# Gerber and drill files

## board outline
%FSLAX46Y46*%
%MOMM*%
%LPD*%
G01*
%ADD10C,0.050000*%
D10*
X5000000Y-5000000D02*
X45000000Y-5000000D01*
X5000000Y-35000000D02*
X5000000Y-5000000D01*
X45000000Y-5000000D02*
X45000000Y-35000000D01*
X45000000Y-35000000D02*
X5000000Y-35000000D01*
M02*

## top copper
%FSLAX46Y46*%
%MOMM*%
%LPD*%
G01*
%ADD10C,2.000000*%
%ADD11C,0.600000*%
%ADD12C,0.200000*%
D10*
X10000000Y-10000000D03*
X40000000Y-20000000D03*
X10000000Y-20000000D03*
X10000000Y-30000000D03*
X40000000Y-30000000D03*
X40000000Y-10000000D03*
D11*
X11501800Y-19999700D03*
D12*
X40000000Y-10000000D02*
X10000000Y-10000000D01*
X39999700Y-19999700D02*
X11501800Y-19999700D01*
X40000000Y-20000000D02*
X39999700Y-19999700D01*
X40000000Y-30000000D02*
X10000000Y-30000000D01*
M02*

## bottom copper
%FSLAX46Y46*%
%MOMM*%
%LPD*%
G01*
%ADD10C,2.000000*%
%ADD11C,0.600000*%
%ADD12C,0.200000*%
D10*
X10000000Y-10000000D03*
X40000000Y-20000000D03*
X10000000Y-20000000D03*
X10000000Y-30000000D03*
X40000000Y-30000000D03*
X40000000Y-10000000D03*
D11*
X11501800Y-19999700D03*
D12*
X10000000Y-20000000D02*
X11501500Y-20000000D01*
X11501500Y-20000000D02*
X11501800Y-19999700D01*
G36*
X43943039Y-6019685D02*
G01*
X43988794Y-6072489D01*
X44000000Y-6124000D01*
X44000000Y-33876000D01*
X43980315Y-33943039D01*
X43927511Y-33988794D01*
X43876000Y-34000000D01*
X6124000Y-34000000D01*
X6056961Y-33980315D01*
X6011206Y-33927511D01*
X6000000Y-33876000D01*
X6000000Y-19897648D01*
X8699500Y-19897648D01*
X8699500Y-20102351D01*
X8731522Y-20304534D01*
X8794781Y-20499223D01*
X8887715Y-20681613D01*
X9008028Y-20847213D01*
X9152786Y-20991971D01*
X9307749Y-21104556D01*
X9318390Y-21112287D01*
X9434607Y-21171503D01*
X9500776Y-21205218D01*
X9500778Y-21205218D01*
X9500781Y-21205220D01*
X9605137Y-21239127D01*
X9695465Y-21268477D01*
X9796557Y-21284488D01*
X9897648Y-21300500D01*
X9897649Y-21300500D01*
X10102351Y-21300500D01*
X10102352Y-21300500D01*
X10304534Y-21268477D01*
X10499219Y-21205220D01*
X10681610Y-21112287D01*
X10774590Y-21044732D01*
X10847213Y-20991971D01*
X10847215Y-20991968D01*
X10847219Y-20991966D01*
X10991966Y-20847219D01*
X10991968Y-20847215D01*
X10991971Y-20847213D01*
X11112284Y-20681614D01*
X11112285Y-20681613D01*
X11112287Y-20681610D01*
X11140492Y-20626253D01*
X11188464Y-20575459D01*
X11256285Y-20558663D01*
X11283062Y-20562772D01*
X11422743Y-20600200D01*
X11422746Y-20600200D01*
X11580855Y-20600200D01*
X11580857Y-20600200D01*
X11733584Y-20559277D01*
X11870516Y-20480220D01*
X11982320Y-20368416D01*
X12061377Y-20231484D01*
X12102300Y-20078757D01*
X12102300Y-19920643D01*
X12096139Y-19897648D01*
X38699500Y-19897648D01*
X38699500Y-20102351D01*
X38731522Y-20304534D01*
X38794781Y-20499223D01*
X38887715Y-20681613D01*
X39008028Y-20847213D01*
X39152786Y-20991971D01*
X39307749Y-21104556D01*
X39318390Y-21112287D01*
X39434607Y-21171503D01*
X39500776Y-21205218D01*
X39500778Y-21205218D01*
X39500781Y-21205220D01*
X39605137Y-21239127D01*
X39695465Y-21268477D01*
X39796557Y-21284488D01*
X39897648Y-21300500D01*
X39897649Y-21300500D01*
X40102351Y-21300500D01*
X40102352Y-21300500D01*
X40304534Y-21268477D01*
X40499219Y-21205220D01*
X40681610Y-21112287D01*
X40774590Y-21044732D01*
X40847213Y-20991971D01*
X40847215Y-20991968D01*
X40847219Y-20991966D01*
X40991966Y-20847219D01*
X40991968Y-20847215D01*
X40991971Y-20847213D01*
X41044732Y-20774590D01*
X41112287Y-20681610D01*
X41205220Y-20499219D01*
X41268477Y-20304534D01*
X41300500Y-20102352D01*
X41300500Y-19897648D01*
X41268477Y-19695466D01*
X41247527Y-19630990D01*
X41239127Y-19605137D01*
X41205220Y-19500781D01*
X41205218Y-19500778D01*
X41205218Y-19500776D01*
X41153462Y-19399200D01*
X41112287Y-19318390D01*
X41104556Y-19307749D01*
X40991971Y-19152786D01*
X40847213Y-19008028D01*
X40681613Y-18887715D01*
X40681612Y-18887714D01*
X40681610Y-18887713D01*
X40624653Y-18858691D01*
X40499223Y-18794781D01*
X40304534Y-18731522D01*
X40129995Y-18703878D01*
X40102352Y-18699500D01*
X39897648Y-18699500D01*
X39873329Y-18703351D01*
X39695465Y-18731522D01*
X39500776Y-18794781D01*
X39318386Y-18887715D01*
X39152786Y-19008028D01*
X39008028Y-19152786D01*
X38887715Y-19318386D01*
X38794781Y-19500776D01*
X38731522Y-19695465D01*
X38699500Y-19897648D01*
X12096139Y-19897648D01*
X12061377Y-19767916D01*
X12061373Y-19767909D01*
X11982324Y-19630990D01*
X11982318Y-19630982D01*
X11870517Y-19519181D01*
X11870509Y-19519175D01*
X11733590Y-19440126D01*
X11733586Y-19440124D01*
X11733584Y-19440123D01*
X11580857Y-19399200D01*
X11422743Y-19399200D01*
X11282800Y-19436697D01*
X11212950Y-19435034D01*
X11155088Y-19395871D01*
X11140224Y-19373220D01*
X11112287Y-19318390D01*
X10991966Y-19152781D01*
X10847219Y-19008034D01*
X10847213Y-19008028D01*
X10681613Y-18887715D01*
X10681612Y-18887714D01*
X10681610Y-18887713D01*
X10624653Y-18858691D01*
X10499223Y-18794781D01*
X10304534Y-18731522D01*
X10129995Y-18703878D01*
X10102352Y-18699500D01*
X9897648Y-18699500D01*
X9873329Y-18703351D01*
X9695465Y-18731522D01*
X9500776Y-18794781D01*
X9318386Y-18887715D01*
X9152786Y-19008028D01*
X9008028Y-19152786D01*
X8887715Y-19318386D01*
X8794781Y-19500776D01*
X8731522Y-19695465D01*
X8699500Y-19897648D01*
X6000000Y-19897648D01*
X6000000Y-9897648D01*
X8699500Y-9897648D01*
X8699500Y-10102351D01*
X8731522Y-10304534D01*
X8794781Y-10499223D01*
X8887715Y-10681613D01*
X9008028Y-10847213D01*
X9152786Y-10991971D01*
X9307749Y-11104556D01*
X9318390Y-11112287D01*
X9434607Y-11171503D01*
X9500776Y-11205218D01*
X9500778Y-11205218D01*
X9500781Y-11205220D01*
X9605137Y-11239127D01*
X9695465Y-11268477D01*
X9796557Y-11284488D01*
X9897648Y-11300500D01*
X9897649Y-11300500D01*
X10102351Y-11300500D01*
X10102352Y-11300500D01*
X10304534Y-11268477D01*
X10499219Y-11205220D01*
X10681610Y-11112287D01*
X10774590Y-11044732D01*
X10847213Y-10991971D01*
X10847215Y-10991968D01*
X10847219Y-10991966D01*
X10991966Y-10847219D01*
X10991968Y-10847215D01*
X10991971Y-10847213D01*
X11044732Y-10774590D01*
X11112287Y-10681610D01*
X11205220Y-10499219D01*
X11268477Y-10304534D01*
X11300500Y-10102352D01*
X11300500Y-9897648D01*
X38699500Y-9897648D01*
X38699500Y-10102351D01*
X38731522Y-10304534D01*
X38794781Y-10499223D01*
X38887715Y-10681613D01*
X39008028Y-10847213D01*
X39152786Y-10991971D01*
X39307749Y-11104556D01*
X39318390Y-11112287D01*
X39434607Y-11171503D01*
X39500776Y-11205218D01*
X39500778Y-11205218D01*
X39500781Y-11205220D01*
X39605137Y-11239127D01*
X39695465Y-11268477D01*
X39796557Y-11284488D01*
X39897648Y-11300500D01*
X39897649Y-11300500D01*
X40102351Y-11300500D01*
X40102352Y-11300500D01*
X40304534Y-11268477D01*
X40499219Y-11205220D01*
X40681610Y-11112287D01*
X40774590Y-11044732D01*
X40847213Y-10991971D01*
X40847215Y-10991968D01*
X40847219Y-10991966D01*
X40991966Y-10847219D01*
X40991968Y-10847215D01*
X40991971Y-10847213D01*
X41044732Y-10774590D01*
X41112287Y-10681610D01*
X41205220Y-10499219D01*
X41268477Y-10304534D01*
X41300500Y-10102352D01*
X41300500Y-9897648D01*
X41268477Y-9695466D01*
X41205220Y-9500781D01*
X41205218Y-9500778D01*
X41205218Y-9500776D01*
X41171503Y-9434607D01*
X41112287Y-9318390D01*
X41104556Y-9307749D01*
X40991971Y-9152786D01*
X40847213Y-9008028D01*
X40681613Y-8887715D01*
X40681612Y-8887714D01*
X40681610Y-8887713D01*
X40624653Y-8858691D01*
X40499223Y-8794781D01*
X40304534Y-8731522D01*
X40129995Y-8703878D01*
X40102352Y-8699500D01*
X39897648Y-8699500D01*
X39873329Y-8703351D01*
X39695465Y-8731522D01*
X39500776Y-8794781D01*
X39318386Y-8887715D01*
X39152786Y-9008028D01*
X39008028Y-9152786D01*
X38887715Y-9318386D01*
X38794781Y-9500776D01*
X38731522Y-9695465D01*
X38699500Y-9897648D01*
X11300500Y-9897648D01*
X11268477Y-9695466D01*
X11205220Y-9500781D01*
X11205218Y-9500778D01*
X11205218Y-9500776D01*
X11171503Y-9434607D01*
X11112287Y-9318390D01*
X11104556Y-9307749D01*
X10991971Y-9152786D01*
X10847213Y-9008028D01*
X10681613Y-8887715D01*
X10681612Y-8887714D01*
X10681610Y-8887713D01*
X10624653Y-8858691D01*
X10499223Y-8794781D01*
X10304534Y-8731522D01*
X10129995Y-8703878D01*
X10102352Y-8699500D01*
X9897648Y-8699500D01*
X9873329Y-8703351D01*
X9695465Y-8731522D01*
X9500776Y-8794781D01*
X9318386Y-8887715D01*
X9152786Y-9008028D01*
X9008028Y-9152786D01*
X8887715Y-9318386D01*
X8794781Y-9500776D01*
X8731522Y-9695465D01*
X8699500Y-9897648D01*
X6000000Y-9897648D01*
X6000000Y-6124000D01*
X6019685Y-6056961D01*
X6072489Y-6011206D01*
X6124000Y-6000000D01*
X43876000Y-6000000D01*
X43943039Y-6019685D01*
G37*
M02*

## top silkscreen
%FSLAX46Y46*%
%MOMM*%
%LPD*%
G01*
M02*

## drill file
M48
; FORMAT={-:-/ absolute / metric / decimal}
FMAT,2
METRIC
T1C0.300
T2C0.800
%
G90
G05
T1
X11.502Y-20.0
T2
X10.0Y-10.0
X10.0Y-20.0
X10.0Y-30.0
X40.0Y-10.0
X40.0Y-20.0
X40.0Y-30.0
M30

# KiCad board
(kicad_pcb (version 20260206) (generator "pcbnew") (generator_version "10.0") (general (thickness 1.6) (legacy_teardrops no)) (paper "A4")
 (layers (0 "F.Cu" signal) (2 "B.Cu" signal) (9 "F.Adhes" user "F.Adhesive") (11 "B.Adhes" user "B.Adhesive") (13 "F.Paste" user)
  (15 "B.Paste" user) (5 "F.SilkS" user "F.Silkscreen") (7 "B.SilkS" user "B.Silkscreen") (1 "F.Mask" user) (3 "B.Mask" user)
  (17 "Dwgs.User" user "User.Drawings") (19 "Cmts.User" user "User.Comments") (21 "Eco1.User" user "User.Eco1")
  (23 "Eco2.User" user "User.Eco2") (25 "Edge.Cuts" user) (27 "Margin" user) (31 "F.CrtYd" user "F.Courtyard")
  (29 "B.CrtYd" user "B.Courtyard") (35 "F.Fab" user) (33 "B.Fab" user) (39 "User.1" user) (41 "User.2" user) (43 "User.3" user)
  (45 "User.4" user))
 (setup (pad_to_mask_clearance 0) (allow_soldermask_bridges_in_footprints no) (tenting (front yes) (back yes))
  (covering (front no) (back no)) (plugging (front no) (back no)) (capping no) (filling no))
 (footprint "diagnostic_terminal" (layer "F.Cu") (at 10 10)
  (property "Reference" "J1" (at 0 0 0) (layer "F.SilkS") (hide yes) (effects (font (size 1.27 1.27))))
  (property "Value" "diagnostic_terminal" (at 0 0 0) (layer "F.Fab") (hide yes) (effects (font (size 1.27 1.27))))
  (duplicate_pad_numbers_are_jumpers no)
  (pad "1" thru_hole circle (at 0 0) (size 2 2) (drill 0.8) (layers "*.Cu") (remove_unused_layers no) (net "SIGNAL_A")))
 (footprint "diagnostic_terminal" (layer "F.Cu") (at 40 20)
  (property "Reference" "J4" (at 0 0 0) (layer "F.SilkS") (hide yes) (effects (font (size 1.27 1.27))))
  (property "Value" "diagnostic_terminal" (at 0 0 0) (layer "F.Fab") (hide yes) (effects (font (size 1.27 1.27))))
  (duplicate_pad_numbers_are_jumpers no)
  (pad "1" thru_hole circle (at 0 0) (size 2 2) (drill 0.8) (layers "*.Cu") (remove_unused_layers no) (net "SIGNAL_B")))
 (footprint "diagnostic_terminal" (layer "F.Cu") (at 10 20)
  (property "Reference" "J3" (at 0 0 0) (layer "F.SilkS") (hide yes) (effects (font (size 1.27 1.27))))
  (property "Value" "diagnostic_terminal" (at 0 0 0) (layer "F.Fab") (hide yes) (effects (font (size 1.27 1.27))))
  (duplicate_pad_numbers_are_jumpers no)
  (pad "1" thru_hole circle (at 0 0) (size 2 2) (drill 0.8) (layers "*.Cu") (remove_unused_layers no) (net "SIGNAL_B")))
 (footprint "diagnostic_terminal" (layer "F.Cu") (at 10 30)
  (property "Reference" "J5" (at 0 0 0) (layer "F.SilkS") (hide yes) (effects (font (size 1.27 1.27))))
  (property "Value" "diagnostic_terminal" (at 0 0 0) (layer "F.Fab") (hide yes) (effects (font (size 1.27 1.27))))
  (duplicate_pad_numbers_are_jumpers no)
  (pad "1" thru_hole circle (at 0 0) (size 2 2) (drill 0.8) (layers "*.Cu") (remove_unused_layers no) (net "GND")))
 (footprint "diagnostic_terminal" (layer "F.Cu") (at 40 30)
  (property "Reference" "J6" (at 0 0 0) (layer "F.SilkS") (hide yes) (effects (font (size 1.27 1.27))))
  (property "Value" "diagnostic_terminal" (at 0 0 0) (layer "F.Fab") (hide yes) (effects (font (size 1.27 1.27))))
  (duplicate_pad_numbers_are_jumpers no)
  (pad "1" thru_hole circle (at 0 0) (size 2 2) (drill 0.8) (layers "*.Cu") (remove_unused_layers no) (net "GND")))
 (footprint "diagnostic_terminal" (layer "F.Cu") (at 40 10)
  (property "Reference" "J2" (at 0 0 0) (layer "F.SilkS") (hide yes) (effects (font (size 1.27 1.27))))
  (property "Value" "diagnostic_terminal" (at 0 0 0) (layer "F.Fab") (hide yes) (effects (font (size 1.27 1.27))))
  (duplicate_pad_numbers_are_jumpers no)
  (pad "1" thru_hole circle (at 0 0) (size 2 2) (drill 0.8) (layers "*.Cu") (remove_unused_layers no) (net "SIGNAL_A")))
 (gr_line (start 5 5) (end 45 5) (stroke (width 0.05) (type default)) (layer "Edge.Cuts"))
 (gr_line (start 5 35) (end 5 5) (stroke (width 0.05) (type default)) (layer "Edge.Cuts"))
 (gr_line (start 45 5) (end 45 35) (stroke (width 0.05) (type default)) (layer "Edge.Cuts"))
 (gr_line (start 45 35) (end 5 35) (stroke (width 0.05) (type default)) (layer "Edge.Cuts"))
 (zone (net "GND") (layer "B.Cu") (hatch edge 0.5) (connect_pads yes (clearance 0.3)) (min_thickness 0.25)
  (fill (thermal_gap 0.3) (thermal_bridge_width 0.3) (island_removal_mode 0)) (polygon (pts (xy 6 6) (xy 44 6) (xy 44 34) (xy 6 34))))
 (segment (start 40 10) (end 10 10) (width 0.2) (layer "F.Cu") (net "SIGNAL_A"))
 (segment (start 39.9997 19.9997) (end 11.5018 19.9997) (width 0.2) (layer "F.Cu") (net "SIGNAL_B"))
 (segment (start 40 20) (end 39.9997 19.9997) (width 0.2) (layer "F.Cu") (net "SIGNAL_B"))
 (via (at 11.5018 19.9997) (size 0.6) (drill 0.3) (layers "F.Cu" "B.Cu") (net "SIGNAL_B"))
 (segment (start 10 20) (end 11.5015 20) (width 0.2) (layer "B.Cu") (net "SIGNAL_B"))
 (segment (start 11.5015 20) (end 11.5018 19.9997) (width 0.2) (layer "B.Cu") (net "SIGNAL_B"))
 (segment (start 40 30) (end 10 30) (width 0.2) (layer "F.Cu") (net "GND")))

